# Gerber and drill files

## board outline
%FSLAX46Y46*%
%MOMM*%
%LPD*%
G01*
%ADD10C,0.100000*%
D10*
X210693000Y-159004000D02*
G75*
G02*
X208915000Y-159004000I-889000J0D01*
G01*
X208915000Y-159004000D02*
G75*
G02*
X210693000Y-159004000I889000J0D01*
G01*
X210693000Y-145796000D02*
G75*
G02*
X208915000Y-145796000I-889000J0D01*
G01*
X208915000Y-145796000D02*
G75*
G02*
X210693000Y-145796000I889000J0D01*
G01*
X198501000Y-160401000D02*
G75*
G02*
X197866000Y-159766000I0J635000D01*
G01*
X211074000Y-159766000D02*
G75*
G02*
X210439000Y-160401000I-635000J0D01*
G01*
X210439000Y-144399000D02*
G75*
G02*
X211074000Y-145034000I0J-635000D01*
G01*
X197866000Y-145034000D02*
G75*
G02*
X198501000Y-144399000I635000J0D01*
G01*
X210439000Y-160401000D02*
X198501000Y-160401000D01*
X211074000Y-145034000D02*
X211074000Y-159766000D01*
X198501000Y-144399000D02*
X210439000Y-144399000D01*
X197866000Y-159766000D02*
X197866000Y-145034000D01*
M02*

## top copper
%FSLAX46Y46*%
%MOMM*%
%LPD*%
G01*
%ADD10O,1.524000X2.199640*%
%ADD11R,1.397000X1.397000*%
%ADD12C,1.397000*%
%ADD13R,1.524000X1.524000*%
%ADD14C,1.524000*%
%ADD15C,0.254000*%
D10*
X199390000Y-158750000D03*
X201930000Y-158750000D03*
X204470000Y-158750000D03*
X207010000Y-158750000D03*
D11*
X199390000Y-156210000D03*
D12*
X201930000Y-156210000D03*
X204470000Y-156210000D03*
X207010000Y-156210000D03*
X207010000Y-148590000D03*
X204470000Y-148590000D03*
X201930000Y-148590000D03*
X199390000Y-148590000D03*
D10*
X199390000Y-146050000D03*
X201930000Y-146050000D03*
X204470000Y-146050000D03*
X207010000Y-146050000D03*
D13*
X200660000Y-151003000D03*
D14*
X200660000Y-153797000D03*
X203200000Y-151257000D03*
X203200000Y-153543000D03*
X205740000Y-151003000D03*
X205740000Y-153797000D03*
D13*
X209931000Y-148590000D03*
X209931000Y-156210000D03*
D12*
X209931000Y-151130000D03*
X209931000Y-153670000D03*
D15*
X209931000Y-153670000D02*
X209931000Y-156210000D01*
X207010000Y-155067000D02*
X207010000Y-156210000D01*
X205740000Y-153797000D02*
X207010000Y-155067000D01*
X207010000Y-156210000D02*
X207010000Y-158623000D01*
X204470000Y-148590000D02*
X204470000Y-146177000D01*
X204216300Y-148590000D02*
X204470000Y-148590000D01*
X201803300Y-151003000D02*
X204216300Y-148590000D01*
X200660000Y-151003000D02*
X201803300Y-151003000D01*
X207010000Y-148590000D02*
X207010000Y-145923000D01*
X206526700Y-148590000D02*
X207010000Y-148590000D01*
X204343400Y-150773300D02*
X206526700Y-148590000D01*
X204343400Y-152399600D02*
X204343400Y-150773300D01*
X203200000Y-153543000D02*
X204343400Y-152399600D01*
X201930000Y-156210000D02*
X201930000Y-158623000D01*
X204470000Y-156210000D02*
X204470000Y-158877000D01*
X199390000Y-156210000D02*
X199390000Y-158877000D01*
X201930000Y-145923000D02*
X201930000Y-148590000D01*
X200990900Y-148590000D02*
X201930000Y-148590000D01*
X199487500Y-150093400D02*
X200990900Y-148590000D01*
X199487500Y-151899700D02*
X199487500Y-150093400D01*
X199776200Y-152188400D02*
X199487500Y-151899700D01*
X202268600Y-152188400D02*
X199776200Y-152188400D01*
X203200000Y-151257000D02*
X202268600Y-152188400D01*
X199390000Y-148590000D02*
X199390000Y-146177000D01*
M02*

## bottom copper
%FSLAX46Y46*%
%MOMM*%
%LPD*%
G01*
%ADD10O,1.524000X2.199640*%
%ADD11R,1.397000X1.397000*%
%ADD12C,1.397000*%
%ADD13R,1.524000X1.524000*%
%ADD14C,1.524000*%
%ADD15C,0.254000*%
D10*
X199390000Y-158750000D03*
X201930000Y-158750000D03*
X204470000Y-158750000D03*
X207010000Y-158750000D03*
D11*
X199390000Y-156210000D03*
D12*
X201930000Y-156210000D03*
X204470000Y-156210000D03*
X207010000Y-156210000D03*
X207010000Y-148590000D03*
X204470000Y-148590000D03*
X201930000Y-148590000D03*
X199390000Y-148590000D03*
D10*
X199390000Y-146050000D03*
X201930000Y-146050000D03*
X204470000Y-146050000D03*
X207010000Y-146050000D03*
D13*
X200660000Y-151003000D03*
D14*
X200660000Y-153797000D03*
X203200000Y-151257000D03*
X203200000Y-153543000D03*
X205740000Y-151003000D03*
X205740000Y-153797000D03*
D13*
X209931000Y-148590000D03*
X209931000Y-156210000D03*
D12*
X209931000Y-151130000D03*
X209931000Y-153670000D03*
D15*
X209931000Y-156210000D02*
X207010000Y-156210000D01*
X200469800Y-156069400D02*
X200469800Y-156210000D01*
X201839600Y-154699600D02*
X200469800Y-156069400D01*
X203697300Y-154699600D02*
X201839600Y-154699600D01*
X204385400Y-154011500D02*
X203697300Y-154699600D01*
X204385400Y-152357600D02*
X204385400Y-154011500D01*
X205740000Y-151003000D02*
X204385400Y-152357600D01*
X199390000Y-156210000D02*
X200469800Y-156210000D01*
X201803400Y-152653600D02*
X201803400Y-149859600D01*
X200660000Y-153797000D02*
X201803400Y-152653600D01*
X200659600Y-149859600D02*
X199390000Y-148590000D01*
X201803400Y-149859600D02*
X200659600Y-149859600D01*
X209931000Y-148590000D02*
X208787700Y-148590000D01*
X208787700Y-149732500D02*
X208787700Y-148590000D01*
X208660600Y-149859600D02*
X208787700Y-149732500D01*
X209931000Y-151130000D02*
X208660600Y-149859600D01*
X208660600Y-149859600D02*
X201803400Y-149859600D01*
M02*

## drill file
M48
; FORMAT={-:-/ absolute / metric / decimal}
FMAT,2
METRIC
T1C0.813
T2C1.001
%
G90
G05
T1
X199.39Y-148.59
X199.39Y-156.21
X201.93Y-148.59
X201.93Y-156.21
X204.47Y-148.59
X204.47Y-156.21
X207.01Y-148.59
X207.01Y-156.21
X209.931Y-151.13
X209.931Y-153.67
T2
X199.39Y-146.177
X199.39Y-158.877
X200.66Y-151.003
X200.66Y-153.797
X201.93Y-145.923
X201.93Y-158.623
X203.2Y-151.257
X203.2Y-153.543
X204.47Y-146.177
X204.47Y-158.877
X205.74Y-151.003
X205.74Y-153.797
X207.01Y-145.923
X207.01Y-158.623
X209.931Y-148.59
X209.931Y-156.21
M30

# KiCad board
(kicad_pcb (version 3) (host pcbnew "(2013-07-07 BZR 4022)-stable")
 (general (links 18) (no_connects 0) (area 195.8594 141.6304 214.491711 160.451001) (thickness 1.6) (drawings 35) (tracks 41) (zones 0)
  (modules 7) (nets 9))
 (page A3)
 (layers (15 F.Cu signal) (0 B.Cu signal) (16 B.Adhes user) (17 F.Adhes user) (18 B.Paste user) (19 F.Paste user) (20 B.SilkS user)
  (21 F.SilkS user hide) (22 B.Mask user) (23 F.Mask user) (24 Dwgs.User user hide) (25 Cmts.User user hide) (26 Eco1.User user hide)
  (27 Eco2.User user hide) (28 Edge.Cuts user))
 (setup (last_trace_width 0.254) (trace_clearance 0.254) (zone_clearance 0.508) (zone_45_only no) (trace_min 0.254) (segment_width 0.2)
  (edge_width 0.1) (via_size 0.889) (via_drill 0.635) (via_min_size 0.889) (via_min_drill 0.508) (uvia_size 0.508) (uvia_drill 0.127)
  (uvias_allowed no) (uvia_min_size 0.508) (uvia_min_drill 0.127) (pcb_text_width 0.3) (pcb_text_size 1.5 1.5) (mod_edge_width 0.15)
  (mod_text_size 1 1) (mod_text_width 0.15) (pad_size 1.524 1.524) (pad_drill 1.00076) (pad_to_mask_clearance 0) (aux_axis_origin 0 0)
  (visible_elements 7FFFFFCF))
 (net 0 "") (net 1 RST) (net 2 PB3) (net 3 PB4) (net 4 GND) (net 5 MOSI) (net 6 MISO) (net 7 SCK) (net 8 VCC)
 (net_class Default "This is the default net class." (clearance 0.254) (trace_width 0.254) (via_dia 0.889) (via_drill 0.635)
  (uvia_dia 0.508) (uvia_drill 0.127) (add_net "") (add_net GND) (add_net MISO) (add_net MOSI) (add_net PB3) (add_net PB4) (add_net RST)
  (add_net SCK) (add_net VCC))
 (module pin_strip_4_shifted (layer F.Cu) (at 203.2 158.75)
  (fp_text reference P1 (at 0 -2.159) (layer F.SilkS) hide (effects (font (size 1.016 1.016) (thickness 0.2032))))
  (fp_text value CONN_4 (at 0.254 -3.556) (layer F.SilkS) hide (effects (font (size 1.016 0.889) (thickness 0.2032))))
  (pad 1 thru_hole oval (at -3.81 0.127) (size 1.524 2.19964) (drill 1.00076 (offset 0 -0.127)) (layers *.Cu *.Mask F.SilkS) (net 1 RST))
  (pad 2 thru_hole oval (at -1.27 -0.127) (size 1.524 2.19964) (drill 1.00076 (offset 0 0.127)) (layers *.Cu *.Mask F.SilkS) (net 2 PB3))
  (pad 3 thru_hole oval (at 1.27 0.127) (size 1.524 2.19964) (drill 1.00076 (offset 0 -0.127)) (layers *.Cu *.Mask F.SilkS) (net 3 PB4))
  (pad 4 thru_hole oval (at 3.81 -0.127) (size 1.524 2.19964) (drill 1.00076 (offset 0 0.127)) (layers *.Cu *.Mask F.SilkS) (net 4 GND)))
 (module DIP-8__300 (layer F.Cu) (at 203.2 152.4)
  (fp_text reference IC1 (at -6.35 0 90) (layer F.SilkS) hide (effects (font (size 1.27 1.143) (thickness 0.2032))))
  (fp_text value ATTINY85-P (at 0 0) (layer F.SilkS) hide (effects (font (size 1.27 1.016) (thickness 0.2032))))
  (pad 1 thru_hole rect (at -3.81 3.81) (size 1.397 1.397) (drill 0.8128) (layers *.Cu *.Mask F.SilkS) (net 1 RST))
  (pad 2 thru_hole circle (at -1.27 3.81) (size 1.397 1.397) (drill 0.8128) (layers *.Cu *.Mask F.SilkS) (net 2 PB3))
  (pad 3 thru_hole circle (at 1.27 3.81) (size 1.397 1.397) (drill 0.8128) (layers *.Cu *.Mask F.SilkS) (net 3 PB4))
  (pad 4 thru_hole circle (at 3.81 3.81) (size 1.397 1.397) (drill 0.8128) (layers *.Cu *.Mask F.SilkS) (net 4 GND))
  (pad 5 thru_hole circle (at 3.81 -3.81) (size 1.397 1.397) (drill 0.8128) (layers *.Cu *.Mask F.SilkS) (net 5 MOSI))
  (pad 6 thru_hole circle (at 1.27 -3.81) (size 1.397 1.397) (drill 0.8128) (layers *.Cu *.Mask F.SilkS) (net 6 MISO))
  (pad 7 thru_hole circle (at -1.27 -3.81) (size 1.397 1.397) (drill 0.8128) (layers *.Cu *.Mask F.SilkS) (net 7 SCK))
  (pad 8 thru_hole circle (at -3.81 -3.81) (size 1.397 1.397) (drill 0.8128) (layers *.Cu *.Mask F.SilkS) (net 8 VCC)))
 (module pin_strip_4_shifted (layer F.Cu) (at 203.2 146.05)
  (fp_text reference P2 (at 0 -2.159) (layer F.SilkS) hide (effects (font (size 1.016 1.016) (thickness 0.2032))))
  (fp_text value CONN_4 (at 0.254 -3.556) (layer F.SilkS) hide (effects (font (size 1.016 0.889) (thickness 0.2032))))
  (pad 1 thru_hole oval (at -3.81 0.127) (size 1.524 2.19964) (drill 1.00076 (offset 0 -0.127)) (layers *.Cu *.Mask F.SilkS) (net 8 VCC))
  (pad 2 thru_hole oval (at -1.27 -0.127) (size 1.524 2.19964) (drill 1.00076 (offset 0 0.127)) (layers *.Cu *.Mask F.SilkS) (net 7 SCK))
  (pad 3 thru_hole oval (at 1.27 0.127) (size 1.524 2.19964) (drill 1.00076 (offset 0 -0.127)) (layers *.Cu *.Mask F.SilkS) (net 6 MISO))
  (pad 4 thru_hole oval (at 3.81 -0.127) (size 1.524 2.19964) (drill 1.00076 (offset 0 0.127)) (layers *.Cu *.Mask F.SilkS) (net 5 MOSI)))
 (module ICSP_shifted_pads (layer B.Cu) (at 203.2 152.4)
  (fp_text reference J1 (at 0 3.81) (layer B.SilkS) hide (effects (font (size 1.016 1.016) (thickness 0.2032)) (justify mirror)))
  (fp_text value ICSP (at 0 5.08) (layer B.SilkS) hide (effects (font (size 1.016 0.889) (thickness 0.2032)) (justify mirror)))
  (pad 1 thru_hole rect (at -2.54 -1.397) (size 1.524 1.524) (drill 1.00076) (layers *.Cu *.Mask B.SilkS) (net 6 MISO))
  (pad 2 thru_hole circle (at -2.54 1.397) (size 1.524 1.524) (drill 1.00076) (layers *.Cu *.Mask B.SilkS) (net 8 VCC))
  (pad 3 thru_hole circle (at 0 -1.143) (size 1.524 1.524) (drill 1.00076) (layers *.Cu *.Mask B.SilkS) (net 7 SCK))
  (pad 4 thru_hole circle (at 0 1.143) (size 1.524 1.524) (drill 1.00076) (layers *.Cu *.Mask B.SilkS) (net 5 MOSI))
  (pad 5 thru_hole circle (at 2.54 -1.397) (size 1.524 1.524) (drill 1.00076) (layers *.Cu *.Mask B.SilkS) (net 1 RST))
  (pad 6 thru_hole circle (at 2.54 1.397) (size 1.524 1.524) (drill 1.00076) (layers *.Cu *.Mask B.SilkS) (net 4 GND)))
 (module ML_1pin (layer F.Cu) (at 209.931 148.59)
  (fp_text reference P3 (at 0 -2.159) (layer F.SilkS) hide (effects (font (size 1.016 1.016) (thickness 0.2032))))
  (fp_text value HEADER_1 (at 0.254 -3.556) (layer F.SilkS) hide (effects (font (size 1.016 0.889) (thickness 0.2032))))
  (pad 1 thru_hole rect (at 0 0) (size 1.524 1.524) (drill 1.00076) (layers *.Cu *.Mask F.SilkS) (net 8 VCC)))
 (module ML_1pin (layer F.Cu) (at 209.931 156.21)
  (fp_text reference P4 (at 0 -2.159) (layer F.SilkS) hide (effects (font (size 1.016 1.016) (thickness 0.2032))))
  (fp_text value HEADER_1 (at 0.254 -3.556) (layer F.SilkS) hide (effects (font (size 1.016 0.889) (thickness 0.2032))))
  (pad 1 thru_hole rect (at 0 0) (size 1.524 1.524) (drill 1.00076) (layers *.Cu *.Mask F.SilkS) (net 4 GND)))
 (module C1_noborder (layer F.Cu) (at 209.931 152.4 270)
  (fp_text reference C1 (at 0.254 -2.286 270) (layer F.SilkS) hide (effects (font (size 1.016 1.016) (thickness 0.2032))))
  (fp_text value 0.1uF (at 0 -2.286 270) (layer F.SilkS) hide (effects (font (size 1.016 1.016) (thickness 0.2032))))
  (pad 1 thru_hole circle (at -1.27 0 270) (size 1.397 1.397) (drill 0.8128) (layers *.Cu *.Mask F.SilkS) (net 8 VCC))
  (pad 2 thru_hole circle (at 1.27 0 270) (size 1.397 1.397) (drill 0.8128) (layers *.Cu *.Mask F.SilkS) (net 4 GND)))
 (gr_circle (center 209.804 159.004) (end 210.693 159.004) (layer Edge.Cuts) (width 0.1))
 (gr_circle (center 209.804 145.796) (end 210.693 145.796) (layer Edge.Cuts) (width 0.1))
 (gr_arc (start 198.501 159.766) (end 198.501 160.401) (angle 90) (layer Edge.Cuts) (width 0.1))
 (gr_arc (start 210.439 159.766) (end 211.074 159.766) (angle 90) (layer Edge.Cuts) (width 0.1))
 (gr_arc (start 210.439 145.034) (end 210.439 144.399) (angle 90) (layer Edge.Cuts) (width 0.1))
 (gr_arc (start 198.501 145.034) (end 197.866 145.034) (angle 90) (layer Edge.Cuts) (width 0.1))
 (gr_line (start 210.439 160.401) (end 198.501 160.401) (angle 90) (layer Edge.Cuts) (width 0.1))
 (gr_line (start 211.074 145.034) (end 211.074 159.766) (angle 90) (layer Edge.Cuts) (width 0.1))
 (gr_line (start 198.501 144.399) (end 210.439 144.399) (angle 90) (layer Edge.Cuts) (width 0.1))
 (gr_line (start 197.866 159.766) (end 197.866 145.034) (angle 90) (layer Edge.Cuts) (width 0.1))
 (segment (start 209.931 153.67) (end 209.931 156.21) (width 0.254) (layer F.Cu) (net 4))
 (segment (start 209.931 156.21) (end 207.01 156.21) (width 0.254) (layer B.Cu) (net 4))
 (segment (start 207.01 155.067) (end 207.01 156.21) (width 0.254) (layer F.Cu) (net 4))
 (segment (start 205.74 153.797) (end 207.01 155.067) (width 0.254) (layer F.Cu) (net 4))
 (segment (start 207.01 156.21) (end 207.01 158.623) (width 0.254) (layer F.Cu) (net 4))
 (segment (start 204.47 148.59) (end 204.47 146.177) (width 0.254) (layer F.Cu) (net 6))
 (segment (start 204.2163 148.59) (end 204.47 148.59) (width 0.254) (layer F.Cu) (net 6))
 (segment (start 201.8033 151.003) (end 204.2163 148.59) (width 0.254) (layer F.Cu) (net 6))
 (segment (start 200.66 151.003) (end 201.8033 151.003) (width 0.254) (layer F.Cu) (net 6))
 (segment (start 207.01 148.59) (end 207.01 145.923) (width 0.254) (layer F.Cu) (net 5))
 (segment (start 206.5267 148.59) (end 207.01 148.59) (width 0.254) (layer F.Cu) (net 5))
 (segment (start 204.3434 150.7733) (end 206.5267 148.59) (width 0.254) (layer F.Cu) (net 5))
 (segment (start 204.3434 152.3996) (end 204.3434 150.7733) (width 0.254) (layer F.Cu) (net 5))
 (segment (start 203.2 153.543) (end 204.3434 152.3996) (width 0.254) (layer F.Cu) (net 5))
 (segment (start 201.93 156.21) (end 201.93 158.623) (width 0.254) (layer F.Cu) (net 2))
 (segment (start 204.47 156.21) (end 204.47 158.877) (width 0.254) (layer F.Cu) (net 3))
 (segment (start 200.4698 156.0694) (end 200.4698 156.21) (width 0.254) (layer B.Cu) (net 1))
 (segment (start 201.8396 154.6996) (end 200.4698 156.0694) (width 0.254) (layer B.Cu) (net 1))
 (segment (start 203.6973 154.6996) (end 201.8396 154.6996) (width 0.254) (layer B.Cu) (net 1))
 (segment (start 204.3854 154.0115) (end 203.6973 154.6996) (width 0.254) (layer B.Cu) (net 1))
 (segment (start 204.3854 152.3576) (end 204.3854 154.0115) (width 0.254) (layer B.Cu) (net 1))
 (segment (start 205.74 151.003) (end 204.3854 152.3576) (width 0.254) (layer B.Cu) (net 1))
 (segment (start 199.39 156.21) (end 200.4698 156.21) (width 0.254) (layer B.Cu) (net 1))
 (segment (start 199.39 156.21) (end 199.39 158.877) (width 0.254) (layer F.Cu) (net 1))
 (segment (start 201.93 145.923) (end 201.93 148.59) (width 0.254) (layer F.Cu) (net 7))
 (segment (start 200.9909 148.59) (end 201.93 148.59) (width 0.254) (layer F.Cu) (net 7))
 (segment (start 199.4875 150.0934) (end 200.9909 148.59) (width 0.254) (layer F.Cu) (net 7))
 (segment (start 199.4875 151.8997) (end 199.4875 150.0934) (width 0.254) (layer F.Cu) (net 7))
 (segment (start 199.7762 152.1884) (end 199.4875 151.8997) (width 0.254) (layer F.Cu) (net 7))
 (segment (start 202.2686 152.1884) (end 199.7762 152.1884) (width 0.254) (layer F.Cu) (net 7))
 (segment (start 203.2 151.257) (end 202.2686 152.1884) (width 0.254) (layer F.Cu) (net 7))
 (segment (start 199.39 148.59) (end 199.39 146.177) (width 0.254) (layer F.Cu) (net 8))
 (segment (start 201.8034 152.6536) (end 201.8034 149.8596) (width 0.254) (layer B.Cu) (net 8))
 (segment (start 200.66 153.797) (end 201.8034 152.6536) (width 0.254) (layer B.Cu) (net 8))
 (segment (start 200.6596 149.8596) (end 199.39 148.59) (width 0.254) (layer B.Cu) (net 8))
 (segment (start 201.8034 149.8596) (end 200.6596 149.8596) (width 0.254) (layer B.Cu) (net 8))
 (segment (start 209.931 148.59) (end 208.7877 148.59) (width 0.254) (layer B.Cu) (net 8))
 (segment (start 208.7877 149.7325) (end 208.7877 148.59) (width 0.254) (layer B.Cu) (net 8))
 (segment (start 208.6606 149.8596) (end 208.7877 149.7325) (width 0.254) (layer B.Cu) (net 8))
 (segment (start 209.931 151.13) (end 208.6606 149.8596) (width 0.254) (layer B.Cu) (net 8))
 (segment (start 208.6606 149.8596) (end 201.8034 149.8596) (width 0.254) (layer B.Cu) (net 8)))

